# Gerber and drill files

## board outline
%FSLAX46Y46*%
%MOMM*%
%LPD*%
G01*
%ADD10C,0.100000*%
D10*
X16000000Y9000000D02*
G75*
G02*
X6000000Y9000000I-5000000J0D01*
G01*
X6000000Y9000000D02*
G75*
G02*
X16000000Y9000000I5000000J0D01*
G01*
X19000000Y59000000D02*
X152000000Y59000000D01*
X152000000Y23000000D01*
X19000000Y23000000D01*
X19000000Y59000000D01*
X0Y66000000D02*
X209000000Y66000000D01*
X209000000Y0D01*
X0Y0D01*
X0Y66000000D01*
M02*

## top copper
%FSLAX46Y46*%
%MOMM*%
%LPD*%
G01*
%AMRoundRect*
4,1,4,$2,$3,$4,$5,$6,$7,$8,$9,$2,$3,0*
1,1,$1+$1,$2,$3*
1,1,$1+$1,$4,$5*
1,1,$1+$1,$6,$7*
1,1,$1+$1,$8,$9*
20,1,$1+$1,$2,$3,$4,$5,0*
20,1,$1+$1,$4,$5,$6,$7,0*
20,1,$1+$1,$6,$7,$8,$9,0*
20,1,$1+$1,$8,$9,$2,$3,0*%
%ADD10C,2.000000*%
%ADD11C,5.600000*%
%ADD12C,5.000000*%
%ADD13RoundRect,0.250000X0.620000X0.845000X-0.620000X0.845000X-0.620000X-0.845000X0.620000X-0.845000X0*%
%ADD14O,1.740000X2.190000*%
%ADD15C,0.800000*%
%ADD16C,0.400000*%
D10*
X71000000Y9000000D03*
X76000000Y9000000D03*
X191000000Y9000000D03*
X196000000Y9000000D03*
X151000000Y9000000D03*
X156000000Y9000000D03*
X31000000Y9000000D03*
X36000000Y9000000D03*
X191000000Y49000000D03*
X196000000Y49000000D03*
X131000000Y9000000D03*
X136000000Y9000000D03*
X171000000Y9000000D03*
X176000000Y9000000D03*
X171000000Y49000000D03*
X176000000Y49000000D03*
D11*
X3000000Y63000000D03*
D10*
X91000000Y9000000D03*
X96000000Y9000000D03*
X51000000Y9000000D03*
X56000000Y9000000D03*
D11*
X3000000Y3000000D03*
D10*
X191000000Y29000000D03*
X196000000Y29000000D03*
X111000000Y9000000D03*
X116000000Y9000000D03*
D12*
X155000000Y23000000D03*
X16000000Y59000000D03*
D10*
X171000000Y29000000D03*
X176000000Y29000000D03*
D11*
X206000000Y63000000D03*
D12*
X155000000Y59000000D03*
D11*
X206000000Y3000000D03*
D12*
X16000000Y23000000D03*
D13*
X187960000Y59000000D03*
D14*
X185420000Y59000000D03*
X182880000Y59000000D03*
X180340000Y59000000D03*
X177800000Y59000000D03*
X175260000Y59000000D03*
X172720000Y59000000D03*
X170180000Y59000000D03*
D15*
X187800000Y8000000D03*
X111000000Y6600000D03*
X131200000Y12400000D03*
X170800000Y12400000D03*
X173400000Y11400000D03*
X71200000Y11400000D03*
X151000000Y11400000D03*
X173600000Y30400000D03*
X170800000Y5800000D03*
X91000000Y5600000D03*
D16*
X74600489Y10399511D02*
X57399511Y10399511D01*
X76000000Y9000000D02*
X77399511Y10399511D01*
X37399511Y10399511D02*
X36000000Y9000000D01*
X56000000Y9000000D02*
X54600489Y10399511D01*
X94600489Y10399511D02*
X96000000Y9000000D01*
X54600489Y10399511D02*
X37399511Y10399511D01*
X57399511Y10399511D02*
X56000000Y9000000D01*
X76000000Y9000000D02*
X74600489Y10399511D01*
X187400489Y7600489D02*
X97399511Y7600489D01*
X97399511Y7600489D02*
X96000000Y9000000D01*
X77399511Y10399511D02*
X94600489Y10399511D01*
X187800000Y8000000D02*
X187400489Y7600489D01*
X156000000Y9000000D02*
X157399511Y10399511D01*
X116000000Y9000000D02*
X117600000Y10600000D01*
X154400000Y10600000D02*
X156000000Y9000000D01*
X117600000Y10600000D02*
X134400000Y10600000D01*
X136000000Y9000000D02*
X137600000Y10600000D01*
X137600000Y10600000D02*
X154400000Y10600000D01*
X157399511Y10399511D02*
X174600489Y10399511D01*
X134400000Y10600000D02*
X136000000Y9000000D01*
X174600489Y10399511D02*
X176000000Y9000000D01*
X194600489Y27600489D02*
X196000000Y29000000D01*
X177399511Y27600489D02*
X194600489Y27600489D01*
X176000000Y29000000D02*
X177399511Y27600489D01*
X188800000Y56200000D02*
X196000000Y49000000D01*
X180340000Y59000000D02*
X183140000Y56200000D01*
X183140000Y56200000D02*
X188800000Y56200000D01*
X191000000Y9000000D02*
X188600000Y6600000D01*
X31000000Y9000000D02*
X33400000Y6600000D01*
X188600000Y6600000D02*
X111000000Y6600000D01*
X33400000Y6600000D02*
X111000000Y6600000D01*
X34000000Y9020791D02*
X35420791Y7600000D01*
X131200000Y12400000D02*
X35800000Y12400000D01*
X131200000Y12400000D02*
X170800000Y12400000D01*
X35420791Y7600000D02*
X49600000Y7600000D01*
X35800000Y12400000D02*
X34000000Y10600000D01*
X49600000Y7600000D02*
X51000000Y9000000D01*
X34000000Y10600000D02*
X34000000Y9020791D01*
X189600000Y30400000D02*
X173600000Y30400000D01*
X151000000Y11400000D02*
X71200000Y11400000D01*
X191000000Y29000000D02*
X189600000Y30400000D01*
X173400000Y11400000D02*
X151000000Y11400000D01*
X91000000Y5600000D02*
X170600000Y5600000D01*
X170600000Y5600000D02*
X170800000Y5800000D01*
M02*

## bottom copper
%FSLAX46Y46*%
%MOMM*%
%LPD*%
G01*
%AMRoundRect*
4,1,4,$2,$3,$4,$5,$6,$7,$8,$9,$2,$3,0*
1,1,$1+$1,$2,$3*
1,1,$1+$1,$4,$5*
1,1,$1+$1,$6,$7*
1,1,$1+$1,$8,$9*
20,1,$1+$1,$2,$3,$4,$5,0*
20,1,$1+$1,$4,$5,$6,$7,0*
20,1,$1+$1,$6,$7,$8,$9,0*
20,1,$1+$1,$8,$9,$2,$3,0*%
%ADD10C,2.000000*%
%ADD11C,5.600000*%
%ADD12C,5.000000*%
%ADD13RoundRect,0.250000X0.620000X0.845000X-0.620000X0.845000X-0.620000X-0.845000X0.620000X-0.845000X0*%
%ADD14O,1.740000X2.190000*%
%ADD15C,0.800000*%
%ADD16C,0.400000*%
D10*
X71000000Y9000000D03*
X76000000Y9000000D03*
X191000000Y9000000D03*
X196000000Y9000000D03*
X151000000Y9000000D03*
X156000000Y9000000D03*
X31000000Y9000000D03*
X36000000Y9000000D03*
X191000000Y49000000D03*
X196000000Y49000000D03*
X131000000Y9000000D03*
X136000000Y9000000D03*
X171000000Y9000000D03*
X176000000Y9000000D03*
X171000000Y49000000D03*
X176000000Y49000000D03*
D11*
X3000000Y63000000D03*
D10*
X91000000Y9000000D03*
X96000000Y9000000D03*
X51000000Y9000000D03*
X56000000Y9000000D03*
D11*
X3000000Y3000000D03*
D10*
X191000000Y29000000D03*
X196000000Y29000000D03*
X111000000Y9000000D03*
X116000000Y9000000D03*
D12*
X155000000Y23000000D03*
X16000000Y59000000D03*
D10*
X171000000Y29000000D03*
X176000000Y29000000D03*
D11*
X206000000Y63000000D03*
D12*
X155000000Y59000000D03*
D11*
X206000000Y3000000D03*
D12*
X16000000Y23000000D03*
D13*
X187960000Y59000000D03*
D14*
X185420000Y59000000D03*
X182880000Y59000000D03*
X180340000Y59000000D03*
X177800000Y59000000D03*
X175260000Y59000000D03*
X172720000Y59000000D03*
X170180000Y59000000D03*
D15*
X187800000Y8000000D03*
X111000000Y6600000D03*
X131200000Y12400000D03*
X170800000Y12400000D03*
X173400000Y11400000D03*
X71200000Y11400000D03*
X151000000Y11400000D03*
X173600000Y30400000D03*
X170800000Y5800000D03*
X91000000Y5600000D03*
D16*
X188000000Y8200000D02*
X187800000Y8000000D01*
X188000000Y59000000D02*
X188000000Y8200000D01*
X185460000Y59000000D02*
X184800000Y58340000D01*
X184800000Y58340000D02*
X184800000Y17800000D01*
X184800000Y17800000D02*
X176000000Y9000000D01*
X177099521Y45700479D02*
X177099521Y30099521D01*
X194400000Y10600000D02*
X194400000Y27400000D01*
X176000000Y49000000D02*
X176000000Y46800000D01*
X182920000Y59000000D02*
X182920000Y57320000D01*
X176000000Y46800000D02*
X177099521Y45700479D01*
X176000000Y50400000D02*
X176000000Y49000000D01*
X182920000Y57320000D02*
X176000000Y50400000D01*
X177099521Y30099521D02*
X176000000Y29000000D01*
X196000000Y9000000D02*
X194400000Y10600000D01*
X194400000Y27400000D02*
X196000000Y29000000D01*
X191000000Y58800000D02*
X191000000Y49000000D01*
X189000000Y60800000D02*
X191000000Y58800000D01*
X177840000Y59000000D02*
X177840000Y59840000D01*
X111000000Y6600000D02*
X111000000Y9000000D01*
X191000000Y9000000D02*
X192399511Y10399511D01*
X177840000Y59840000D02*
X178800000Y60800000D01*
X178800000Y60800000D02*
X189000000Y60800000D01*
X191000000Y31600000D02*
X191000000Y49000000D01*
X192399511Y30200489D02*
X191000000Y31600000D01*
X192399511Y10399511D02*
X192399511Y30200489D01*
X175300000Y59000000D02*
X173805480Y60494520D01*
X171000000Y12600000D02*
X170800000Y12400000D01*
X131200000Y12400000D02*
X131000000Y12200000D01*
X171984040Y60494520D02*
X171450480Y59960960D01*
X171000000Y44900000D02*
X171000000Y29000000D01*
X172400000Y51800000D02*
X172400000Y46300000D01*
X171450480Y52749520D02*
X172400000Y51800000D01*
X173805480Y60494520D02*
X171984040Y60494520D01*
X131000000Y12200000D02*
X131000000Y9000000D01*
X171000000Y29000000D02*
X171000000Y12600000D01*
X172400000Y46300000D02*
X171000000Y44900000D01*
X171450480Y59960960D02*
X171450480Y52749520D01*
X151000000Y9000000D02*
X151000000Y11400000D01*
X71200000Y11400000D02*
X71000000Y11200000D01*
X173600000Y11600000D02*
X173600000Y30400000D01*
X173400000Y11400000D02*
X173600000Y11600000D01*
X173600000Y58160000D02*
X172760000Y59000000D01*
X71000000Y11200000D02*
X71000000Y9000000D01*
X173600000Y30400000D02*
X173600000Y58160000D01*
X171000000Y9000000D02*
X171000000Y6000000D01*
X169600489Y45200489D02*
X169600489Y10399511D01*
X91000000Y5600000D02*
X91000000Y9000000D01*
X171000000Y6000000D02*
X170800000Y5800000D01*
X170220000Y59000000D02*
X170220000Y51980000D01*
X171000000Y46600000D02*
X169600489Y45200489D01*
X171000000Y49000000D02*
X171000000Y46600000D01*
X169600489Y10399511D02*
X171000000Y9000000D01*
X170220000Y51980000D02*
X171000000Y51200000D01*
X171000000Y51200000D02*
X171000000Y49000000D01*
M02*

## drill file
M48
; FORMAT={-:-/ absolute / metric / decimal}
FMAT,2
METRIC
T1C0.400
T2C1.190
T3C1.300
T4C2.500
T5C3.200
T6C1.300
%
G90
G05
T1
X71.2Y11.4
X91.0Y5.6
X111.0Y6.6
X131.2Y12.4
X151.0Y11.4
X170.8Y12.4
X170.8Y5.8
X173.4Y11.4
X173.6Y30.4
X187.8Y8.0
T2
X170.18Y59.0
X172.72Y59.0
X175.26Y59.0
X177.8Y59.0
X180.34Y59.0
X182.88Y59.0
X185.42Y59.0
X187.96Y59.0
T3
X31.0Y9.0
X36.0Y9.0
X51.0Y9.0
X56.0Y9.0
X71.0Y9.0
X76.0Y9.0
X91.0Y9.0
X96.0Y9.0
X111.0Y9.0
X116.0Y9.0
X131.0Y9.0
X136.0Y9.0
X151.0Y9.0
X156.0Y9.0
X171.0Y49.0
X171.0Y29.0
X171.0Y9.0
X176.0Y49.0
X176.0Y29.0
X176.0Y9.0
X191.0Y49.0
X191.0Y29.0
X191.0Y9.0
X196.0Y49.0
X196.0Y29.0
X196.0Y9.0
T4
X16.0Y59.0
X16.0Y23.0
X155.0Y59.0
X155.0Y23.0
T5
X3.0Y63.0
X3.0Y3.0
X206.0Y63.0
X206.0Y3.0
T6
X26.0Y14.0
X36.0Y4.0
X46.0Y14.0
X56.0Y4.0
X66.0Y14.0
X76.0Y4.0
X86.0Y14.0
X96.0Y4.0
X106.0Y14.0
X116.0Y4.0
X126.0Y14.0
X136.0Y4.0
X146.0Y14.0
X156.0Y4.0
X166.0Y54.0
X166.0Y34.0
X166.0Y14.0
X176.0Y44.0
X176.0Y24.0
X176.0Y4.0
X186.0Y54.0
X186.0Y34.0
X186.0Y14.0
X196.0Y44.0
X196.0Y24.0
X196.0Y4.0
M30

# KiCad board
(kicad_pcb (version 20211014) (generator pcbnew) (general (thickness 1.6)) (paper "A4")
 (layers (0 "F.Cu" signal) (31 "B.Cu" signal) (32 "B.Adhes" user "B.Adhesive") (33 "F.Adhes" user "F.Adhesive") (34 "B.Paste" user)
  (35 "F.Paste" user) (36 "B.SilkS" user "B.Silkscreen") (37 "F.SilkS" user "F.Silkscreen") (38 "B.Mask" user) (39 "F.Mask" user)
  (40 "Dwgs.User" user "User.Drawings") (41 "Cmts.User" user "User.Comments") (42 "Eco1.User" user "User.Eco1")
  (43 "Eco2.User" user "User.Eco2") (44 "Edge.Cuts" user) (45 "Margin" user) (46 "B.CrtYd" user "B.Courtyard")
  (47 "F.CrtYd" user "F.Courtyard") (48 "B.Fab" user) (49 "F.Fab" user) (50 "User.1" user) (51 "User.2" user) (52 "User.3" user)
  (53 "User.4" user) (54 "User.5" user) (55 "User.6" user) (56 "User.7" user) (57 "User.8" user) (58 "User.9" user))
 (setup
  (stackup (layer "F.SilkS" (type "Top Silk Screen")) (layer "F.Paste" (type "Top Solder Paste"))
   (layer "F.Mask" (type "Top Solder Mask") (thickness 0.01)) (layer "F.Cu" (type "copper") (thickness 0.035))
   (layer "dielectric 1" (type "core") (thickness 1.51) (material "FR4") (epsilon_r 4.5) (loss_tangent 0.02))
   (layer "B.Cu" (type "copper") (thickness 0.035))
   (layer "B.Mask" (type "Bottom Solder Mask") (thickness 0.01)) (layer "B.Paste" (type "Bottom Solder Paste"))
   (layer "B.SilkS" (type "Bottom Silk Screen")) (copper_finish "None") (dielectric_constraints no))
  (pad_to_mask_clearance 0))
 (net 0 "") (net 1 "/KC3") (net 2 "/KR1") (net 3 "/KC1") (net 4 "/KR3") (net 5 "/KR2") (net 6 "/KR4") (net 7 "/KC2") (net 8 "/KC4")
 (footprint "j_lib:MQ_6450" (layer "F.Cu") (at 71 -9)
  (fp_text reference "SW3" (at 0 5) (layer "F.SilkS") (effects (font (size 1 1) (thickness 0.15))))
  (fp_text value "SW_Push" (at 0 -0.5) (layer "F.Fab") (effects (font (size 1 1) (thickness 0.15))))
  (pad "" np_thru_hole circle locked (at -5 -5) (size 1.3 1.3) (drill 1.3) (layers *.Cu *.Mask))
  (pad "" np_thru_hole circle locked (at 5 5) (size 1.3 1.3) (drill 1.3) (layers *.Cu *.Mask))
  (pad "1" thru_hole circle locked (at 0 0) (size 2 2) (drill 1.3) (layers *.Cu *.Mask) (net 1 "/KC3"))
  (pad "2" thru_hole circle locked (at 5 0) (size 2 2) (drill 1.3) (layers *.Cu *.Mask) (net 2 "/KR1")))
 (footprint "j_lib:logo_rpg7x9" (layer "F.Cu") (at 158.2 -39.4)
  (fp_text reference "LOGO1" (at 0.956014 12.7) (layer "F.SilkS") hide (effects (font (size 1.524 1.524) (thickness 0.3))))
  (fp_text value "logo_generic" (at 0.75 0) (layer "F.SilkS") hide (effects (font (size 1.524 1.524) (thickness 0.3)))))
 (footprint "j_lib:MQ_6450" (layer "F.Cu") (at 191 -9)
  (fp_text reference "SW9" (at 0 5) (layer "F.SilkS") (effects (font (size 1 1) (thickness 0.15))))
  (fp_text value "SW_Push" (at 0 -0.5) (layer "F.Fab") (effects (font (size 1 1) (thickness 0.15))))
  (pad "" np_thru_hole circle locked (at 5 5) (size 1.3 1.3) (drill 1.3) (layers *.Cu *.Mask))
  (pad "" np_thru_hole circle locked (at -5 -5) (size 1.3 1.3) (drill 1.3) (layers *.Cu *.Mask))
  (pad "1" thru_hole circle locked (at 0 0) (size 2 2) (drill 1.3) (layers *.Cu *.Mask) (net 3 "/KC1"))
  (pad "2" thru_hole circle locked (at 5 0) (size 2 2) (drill 1.3) (layers *.Cu *.Mask) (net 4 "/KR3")))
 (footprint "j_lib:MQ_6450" (layer "F.Cu") (at 151 -9)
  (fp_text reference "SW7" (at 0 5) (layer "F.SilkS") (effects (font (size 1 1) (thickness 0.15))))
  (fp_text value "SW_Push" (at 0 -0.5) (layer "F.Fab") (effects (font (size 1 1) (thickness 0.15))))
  (pad "" np_thru_hole circle locked (at 5 5) (size 1.3 1.3) (drill 1.3) (layers *.Cu *.Mask))
  (pad "" np_thru_hole circle locked (at -5 -5) (size 1.3 1.3) (drill 1.3) (layers *.Cu *.Mask))
  (pad "1" thru_hole circle locked (at 0 0) (size 2 2) (drill 1.3) (layers *.Cu *.Mask) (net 1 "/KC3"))
  (pad "2" thru_hole circle locked (at 5 0) (size 2 2) (drill 1.3) (layers *.Cu *.Mask) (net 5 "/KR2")))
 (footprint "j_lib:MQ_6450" (layer "F.Cu") (at 31 -9)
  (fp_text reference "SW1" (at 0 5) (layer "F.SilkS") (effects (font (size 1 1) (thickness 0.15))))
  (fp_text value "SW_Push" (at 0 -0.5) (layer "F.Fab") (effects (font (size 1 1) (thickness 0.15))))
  (pad "" np_thru_hole circle locked (at 5 5) (size 1.3 1.3) (drill 1.3) (layers *.Cu *.Mask))
  (pad "" np_thru_hole circle locked (at -5 -5) (size 1.3 1.3) (drill 1.3) (layers *.Cu *.Mask))
  (pad "1" thru_hole circle locked (at 0 0) (size 2 2) (drill 1.3) (layers *.Cu *.Mask) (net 3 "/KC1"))
  (pad "2" thru_hole circle locked (at 5 0) (size 2 2) (drill 1.3) (layers *.Cu *.Mask) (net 2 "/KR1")))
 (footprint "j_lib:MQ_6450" (layer "F.Cu") (at 191 -49)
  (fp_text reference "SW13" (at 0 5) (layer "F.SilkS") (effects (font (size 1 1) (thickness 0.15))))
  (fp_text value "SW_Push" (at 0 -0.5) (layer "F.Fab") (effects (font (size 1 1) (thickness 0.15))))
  (pad "" np_thru_hole circle locked (at -5 -5) (size 1.3 1.3) (drill 1.3) (layers *.Cu *.Mask))
  (pad "" np_thru_hole circle locked (at 5 5) (size 1.3 1.3) (drill 1.3) (layers *.Cu *.Mask))
  (pad "1" thru_hole circle locked (at 0 0) (size 2 2) (drill 1.3) (layers *.Cu *.Mask) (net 3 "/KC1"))
  (pad "2" thru_hole circle locked (at 5 0) (size 2 2) (drill 1.3) (layers *.Cu *.Mask) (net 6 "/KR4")))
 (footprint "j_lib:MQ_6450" (layer "F.Cu") (at 131 -9)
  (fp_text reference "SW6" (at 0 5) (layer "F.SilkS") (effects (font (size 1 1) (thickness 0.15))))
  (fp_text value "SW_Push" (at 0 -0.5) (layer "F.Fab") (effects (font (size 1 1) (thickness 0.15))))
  (pad "" np_thru_hole circle locked (at 5 5) (size 1.3 1.3) (drill 1.3) (layers *.Cu *.Mask))
  (pad "" np_thru_hole circle locked (at -5 -5) (size 1.3 1.3) (drill 1.3) (layers *.Cu *.Mask))
  (pad "1" thru_hole circle locked (at 0 0) (size 2 2) (drill 1.3) (layers *.Cu *.Mask) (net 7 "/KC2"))
  (pad "2" thru_hole circle locked (at 5 0) (size 2 2) (drill 1.3) (layers *.Cu *.Mask) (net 5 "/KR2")))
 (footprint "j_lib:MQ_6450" (layer "F.Cu") (at 171 -9)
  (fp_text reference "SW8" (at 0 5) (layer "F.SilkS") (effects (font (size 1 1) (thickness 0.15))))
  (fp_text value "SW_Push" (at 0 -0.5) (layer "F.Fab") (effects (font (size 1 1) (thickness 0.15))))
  (pad "" np_thru_hole circle locked (at -5 -5) (size 1.3 1.3) (drill 1.3) (layers *.Cu *.Mask))
  (pad "" np_thru_hole circle locked (at 5 5) (size 1.3 1.3) (drill 1.3) (layers *.Cu *.Mask))
  (pad "1" thru_hole circle locked (at 0 0) (size 2 2) (drill 1.3) (layers *.Cu *.Mask) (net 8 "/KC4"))
  (pad "2" thru_hole circle locked (at 5 0) (size 2 2) (drill 1.3) (layers *.Cu *.Mask) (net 5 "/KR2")))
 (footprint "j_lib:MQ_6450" (layer "F.Cu") (at 171 -49)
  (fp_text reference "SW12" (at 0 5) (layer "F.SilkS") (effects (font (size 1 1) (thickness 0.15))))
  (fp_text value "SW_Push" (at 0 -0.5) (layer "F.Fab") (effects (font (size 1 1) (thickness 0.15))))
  (pad "" np_thru_hole circle locked (at 5 5) (size 1.3 1.3) (drill 1.3) (layers *.Cu *.Mask))
  (pad "" np_thru_hole circle locked (at -5 -5) (size 1.3 1.3) (drill 1.3) (layers *.Cu *.Mask))
  (pad "1" thru_hole circle locked (at 0 0) (size 2 2) (drill 1.3) (layers *.Cu *.Mask) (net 8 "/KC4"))
  (pad "2" thru_hole circle locked (at 5 0) (size 2 2) (drill 1.3) (layers *.Cu *.Mask) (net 4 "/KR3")))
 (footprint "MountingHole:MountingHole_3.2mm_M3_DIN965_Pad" (layer "F.Cu") (at 3 -63)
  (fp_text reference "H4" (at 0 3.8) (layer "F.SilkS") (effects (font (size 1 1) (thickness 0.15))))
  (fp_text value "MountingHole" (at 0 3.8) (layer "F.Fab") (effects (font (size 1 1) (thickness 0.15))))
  (pad "1" thru_hole circle locked (at 0 0) (size 5.6 5.6) (drill 3.2) (layers *.Cu *.Mask)))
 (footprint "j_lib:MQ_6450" (layer "F.Cu") (at 91 -9)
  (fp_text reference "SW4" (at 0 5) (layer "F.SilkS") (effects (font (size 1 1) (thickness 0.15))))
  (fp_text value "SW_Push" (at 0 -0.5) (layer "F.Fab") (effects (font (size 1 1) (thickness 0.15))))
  (pad "" np_thru_hole circle locked (at -5 -5) (size 1.3 1.3) (drill 1.3) (layers *.Cu *.Mask))
  (pad "" np_thru_hole circle locked (at 5 5) (size 1.3 1.3) (drill 1.3) (layers *.Cu *.Mask))
  (pad "1" thru_hole circle locked (at 0 0) (size 2 2) (drill 1.3) (layers *.Cu *.Mask) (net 8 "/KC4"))
  (pad "2" thru_hole circle locked (at 5 0) (size 2 2) (drill 1.3) (layers *.Cu *.Mask) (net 2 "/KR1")))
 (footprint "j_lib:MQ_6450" (layer "F.Cu") (at 51 -9)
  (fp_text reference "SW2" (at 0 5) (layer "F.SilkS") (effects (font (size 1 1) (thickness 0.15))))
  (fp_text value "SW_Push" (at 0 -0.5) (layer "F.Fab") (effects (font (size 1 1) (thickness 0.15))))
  (pad "" np_thru_hole circle locked (at -5 -5) (size 1.3 1.3) (drill 1.3) (layers *.Cu *.Mask))
  (pad "" np_thru_hole circle locked (at 5 5) (size 1.3 1.3) (drill 1.3) (layers *.Cu *.Mask))
  (pad "1" thru_hole circle locked (at 0 0) (size 2 2) (drill 1.3) (layers *.Cu *.Mask) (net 7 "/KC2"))
  (pad "2" thru_hole circle locked (at 5 0) (size 2 2) (drill 1.3) (layers *.Cu *.Mask) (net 2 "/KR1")))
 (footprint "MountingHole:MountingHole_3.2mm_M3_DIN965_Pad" (layer "F.Cu") (at 3 -3)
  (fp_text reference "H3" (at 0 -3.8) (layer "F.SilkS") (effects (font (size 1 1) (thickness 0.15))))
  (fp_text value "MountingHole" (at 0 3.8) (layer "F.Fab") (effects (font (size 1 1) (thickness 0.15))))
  (pad "1" thru_hole circle locked (at 0 0) (size 5.6 5.6) (drill 3.2) (layers *.Cu *.Mask)))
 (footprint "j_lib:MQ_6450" (layer "F.Cu") (at 191 -29)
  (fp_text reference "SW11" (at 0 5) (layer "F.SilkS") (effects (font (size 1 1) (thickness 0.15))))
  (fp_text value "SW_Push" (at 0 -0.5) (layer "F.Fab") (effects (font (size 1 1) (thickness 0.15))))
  (pad "" np_thru_hole circle locked (at 5 5) (size 1.3 1.3) (drill 1.3) (layers *.Cu *.Mask))
  (pad "" np_thru_hole circle locked (at -5 -5) (size 1.3 1.3) (drill 1.3) (layers *.Cu *.Mask))
  (pad "1" thru_hole circle locked (at 0 0) (size 2 2) (drill 1.3) (layers *.Cu *.Mask) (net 1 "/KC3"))
  (pad "2" thru_hole circle locked (at 5 0) (size 2 2) (drill 1.3) (layers *.Cu *.Mask) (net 4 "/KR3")))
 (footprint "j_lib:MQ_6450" (layer "F.Cu") (at 111 -9)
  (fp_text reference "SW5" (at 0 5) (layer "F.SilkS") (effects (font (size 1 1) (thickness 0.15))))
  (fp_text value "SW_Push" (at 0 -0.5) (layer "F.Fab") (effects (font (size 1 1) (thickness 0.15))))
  (pad "" np_thru_hole circle locked (at 5 5) (size 1.3 1.3) (drill 1.3) (layers *.Cu *.Mask))
  (pad "" np_thru_hole circle locked (at -5 -5) (size 1.3 1.3) (drill 1.3) (layers *.Cu *.Mask))
  (pad "1" thru_hole circle locked (at 0 0) (size 2 2) (drill 1.3) (layers *.Cu *.Mask) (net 3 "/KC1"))
  (pad "2" thru_hole circle locked (at 5 0) (size 2 2) (drill 1.3) (layers *.Cu *.Mask) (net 5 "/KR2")))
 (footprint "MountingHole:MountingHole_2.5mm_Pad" (layer "F.Cu") (at 155 -23)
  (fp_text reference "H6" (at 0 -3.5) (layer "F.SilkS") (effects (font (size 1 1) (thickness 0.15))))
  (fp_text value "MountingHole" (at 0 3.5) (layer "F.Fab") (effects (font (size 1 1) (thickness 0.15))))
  (pad "1" thru_hole circle locked (at 0 0) (size 5 5) (drill 2.5) (layers *.Cu *.Mask)))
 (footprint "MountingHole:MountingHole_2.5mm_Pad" (layer "F.Cu") (at 16 -59)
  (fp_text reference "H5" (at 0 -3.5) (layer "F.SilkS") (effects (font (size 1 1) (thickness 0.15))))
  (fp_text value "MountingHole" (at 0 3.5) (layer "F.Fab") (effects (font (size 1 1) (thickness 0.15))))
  (pad "1" thru_hole circle locked (at 0 0) (size 5 5) (drill 2.5) (layers *.Cu *.Mask)))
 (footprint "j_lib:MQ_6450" (layer "F.Cu") (at 171 -29)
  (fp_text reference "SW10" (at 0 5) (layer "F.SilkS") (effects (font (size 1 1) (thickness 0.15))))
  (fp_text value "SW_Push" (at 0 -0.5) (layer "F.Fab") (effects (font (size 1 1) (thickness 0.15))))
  (pad "" np_thru_hole circle locked (at 5 5) (size 1.3 1.3) (drill 1.3) (layers *.Cu *.Mask))
  (pad "" np_thru_hole circle locked (at -5 -5) (size 1.3 1.3) (drill 1.3) (layers *.Cu *.Mask))
  (pad "1" thru_hole circle locked (at 0 0) (size 2 2) (drill 1.3) (layers *.Cu *.Mask) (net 7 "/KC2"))
  (pad "2" thru_hole circle locked (at 5 0) (size 2 2) (drill 1.3) (layers *.Cu *.Mask) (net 4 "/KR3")))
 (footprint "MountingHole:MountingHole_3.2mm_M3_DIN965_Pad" (layer "F.Cu") (at 206 -63)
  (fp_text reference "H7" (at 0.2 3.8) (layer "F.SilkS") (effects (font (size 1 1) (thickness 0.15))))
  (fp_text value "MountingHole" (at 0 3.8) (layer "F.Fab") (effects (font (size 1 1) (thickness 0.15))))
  (pad "1" thru_hole circle locked (at 0 0) (size 5.6 5.6) (drill 3.2) (layers *.Cu *.Mask)))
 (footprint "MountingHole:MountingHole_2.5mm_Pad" (layer "F.Cu") (at 155 -59)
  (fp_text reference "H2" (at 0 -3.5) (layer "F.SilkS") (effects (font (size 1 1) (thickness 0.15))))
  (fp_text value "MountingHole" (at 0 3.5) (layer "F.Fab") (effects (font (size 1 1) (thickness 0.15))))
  (pad "1" thru_hole circle locked (at 0 0) (size 5 5) (drill 2.5) (layers *.Cu *.Mask)))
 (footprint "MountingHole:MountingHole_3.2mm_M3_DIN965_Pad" (layer "F.Cu") (at 206 -3)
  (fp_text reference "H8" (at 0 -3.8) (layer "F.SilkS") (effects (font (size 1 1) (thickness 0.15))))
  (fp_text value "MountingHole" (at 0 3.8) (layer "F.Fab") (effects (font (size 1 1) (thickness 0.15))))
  (pad "1" thru_hole circle locked (at 0 0) (size 5.6 5.6) (drill 3.2) (layers *.Cu *.Mask)))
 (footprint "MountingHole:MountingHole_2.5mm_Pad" (layer "F.Cu") (at 16 -23)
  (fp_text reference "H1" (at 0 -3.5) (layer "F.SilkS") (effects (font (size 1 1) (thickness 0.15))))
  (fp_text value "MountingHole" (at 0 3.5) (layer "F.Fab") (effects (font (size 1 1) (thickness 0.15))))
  (pad "1" thru_hole circle locked (at 0 0) (size 5 5) (drill 2.5) (layers *.Cu *.Mask)))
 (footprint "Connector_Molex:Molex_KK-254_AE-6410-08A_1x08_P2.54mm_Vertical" (layer "B.Cu") (at 187.96 -59 180)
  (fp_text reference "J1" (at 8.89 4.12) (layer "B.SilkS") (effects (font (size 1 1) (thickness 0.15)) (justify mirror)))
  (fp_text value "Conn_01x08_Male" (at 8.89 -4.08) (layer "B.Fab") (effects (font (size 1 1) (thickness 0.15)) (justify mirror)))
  (pad "1" thru_hole roundrect locked (at 0 0 180) (size 1.74 2.19) (drill 1.19) (layers *.Cu *.Mask) (roundrect_rratio 0.1436781609)
   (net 2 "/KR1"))
  (pad "2" thru_hole oval locked (at 2.54 0 180) (size 1.74 2.19) (drill 1.19) (layers *.Cu *.Mask) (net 5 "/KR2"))
  (pad "3" thru_hole oval locked (at 5.08 0 180) (size 1.74 2.19) (drill 1.19) (layers *.Cu *.Mask) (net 4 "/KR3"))
  (pad "4" thru_hole oval locked (at 7.62 0 180) (size 1.74 2.19) (drill 1.19) (layers *.Cu *.Mask) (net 6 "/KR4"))
  (pad "5" thru_hole oval locked (at 10.16 0 180) (size 1.74 2.19) (drill 1.19) (layers *.Cu *.Mask) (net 3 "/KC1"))
  (pad "6" thru_hole oval locked (at 12.7 0 180) (size 1.74 2.19) (drill 1.19) (layers *.Cu *.Mask) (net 7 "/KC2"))
  (pad "7" thru_hole oval locked (at 15.24 0 180) (size 1.74 2.19) (drill 1.19) (layers *.Cu *.Mask) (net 1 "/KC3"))
  (pad "8" thru_hole oval locked (at 17.78 0 180) (size 1.74 2.19) (drill 1.19) (layers *.Cu *.Mask) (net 8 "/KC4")))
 (gr_circle (center 11 -9) (end 16 -9) (layer "Edge.Cuts") (width 0.1) (fill none))
 (gr_rect (start 19 -23) (end 152 -59) (layer "Edge.Cuts") (width 0.1) (fill none))
 (gr_rect (start 0 0) (end 209 -66) (layer "Edge.Cuts") (width 0.1) (fill none))
 (segment (start 74.600489 -10.399511) (end 57.399511 -10.399511) (width 0.4) (layer "F.Cu") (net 2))
 (segment (start 76 -9) (end 77.399511 -10.399511) (width 0.4) (layer "F.Cu") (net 2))
 (segment (start 37.399511 -10.399511) (end 36 -9) (width 0.4) (layer "F.Cu") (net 2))
 (segment (start 56 -9) (end 54.600489 -10.399511) (width 0.4) (layer "F.Cu") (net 2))
 (segment (start 94.600489 -10.399511) (end 96 -9) (width 0.4) (layer "F.Cu") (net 2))
 (segment (start 54.600489 -10.399511) (end 37.399511 -10.399511) (width 0.4) (layer "F.Cu") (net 2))
 (segment (start 57.399511 -10.399511) (end 56 -9) (width 0.4) (layer "F.Cu") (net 2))
 (segment (start 76 -9) (end 74.600489 -10.399511) (width 0.4) (layer "F.Cu") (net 2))
 (segment (start 187.400489 -7.600489) (end 97.399511 -7.600489) (width 0.4) (layer "F.Cu") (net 2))
 (segment (start 97.399511 -7.600489) (end 96 -9) (width 0.4) (layer "F.Cu") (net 2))
 (segment (start 77.399511 -10.399511) (end 94.600489 -10.399511) (width 0.4) (layer "F.Cu") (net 2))
 (segment (start 187.8 -8) (end 187.400489 -7.600489) (width 0.4) (layer "F.Cu") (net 2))
 (via (at 187.8 -8) (size 0.8) (drill 0.4) (layers "F.Cu" "B.Cu") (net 2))
 (segment (start 188 -8.2) (end 187.8 -8) (width 0.4) (layer "B.Cu") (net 2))
 (segment (start 188 -59) (end 188 -8.2) (width 0.4) (layer "B.Cu") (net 2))
 (segment (start 156 -9) (end 157.399511 -10.399511) (width 0.4) (layer "F.Cu") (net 5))
 (segment (start 116 -9) (end 117.6 -10.6) (width 0.4) (layer "F.Cu") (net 5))
 (segment (start 154.4 -10.6) (end 156 -9) (width 0.4) (layer "F.Cu") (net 5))
 (segment (start 117.6 -10.6) (end 134.4 -10.6) (width 0.4) (layer "F.Cu") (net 5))
 (segment (start 136 -9) (end 137.6 -10.6) (width 0.4) (layer "F.Cu") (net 5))
 (segment (start 137.6 -10.6) (end 154.4 -10.6) (width 0.4) (layer "F.Cu") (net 5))
 (segment (start 157.399511 -10.399511) (end 174.600489 -10.399511) (width 0.4) (layer "F.Cu") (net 5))
 (segment (start 134.4 -10.6) (end 136 -9) (width 0.4) (layer "F.Cu") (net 5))
 (segment (start 174.600489 -10.399511) (end 176 -9) (width 0.4) (layer "F.Cu") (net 5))
 (segment (start 185.46 -59) (end 184.8 -58.34) (width 0.4) (layer "B.Cu") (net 5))
 (segment (start 184.8 -58.34) (end 184.8 -17.8) (width 0.4) (layer "B.Cu") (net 5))
 (segment (start 184.8 -17.8) (end 176 -9) (width 0.4) (layer "B.Cu") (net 5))
 (segment (start 194.600489 -27.600489) (end 196 -29) (width 0.4) (layer "F.Cu") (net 4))
 (segment (start 177.399511 -27.600489) (end 194.600489 -27.600489) (width 0.4) (layer "F.Cu") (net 4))
 (segment (start 176 -29) (end 177.399511 -27.600489) (width 0.4) (layer "F.Cu") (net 4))
 (segment (start 177.099521 -45.700479) (end 177.099521 -30.099521) (width 0.4) (layer "B.Cu") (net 4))
 (segment (start 194.4 -10.6) (end 194.4 -27.4) (width 0.4) (layer "B.Cu") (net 4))
 (segment (start 176 -49) (end 176 -46.8) (width 0.4) (layer "B.Cu") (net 4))
 (segment (start 182.92 -59) (end 182.92 -57.32) (width 0.4) (layer "B.Cu") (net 4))
 (segment (start 176 -46.8) (end 177.099521 -45.700479) (width 0.4) (layer "B.Cu") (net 4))
 (segment (start 176 -50.4) (end 176 -49) (width 0.4) (layer "B.Cu") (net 4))
 (segment (start 182.92 -57.32) (end 176 -50.4) (width 0.4) (layer "B.Cu") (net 4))
 (segment (start 177.099521 -30.099521) (end 176 -29) (width 0.4) (layer "B.Cu") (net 4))
 (segment (start 196 -9) (end 194.4 -10.6) (width 0.4) (layer "B.Cu") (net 4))
 (segment (start 194.4 -27.4) (end 196 -29) (width 0.4) (layer "B.Cu") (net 4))
 (segment (start 188.8 -56.2) (end 196 -49) (width 0.4) (layer "F.Cu") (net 6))
 (segment (start 180.34 -59) (end 183.14 -56.2) (width 0.4) (layer "F.Cu") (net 6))
 (segment (start 183.14 -56.2) (end 188.8 -56.2) (width 0.4) (layer "F.Cu") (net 6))
 (segment (start 191 -9) (end 188.6 -6.6) (width 0.4) (layer "F.Cu") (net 3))
 (segment (start 31 -9) (end 33.4 -6.6) (width 0.4) (layer "F.Cu") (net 3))
 (segment (start 188.6 -6.6) (end 111 -6.6) (width 0.4) (layer "F.Cu") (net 3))
 (segment (start 33.4 -6.6) (end 111 -6.6) (width 0.4) (layer "F.Cu") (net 3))
 (via (at 111 -6.6) (size 0.8) (drill 0.4) (layers "F.Cu" "B.Cu") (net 3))
 (segment (start 191 -58.8) (end 191 -49) (width 0.4) (layer "B.Cu") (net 3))
 (segment (start 189 -60.8) (end 191 -58.8) (width 0.4) (layer "B.Cu") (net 3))
 (segment (start 177.84 -59) (end 177.84 -59.84) (width 0.4) (layer "B.Cu") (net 3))
 (segment (start 111 -6.6) (end 111 -9) (width 0.4) (layer "B.Cu") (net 3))
 (segment (start 191 -9) (end 192.399511 -10.399511) (width 0.4) (layer "B.Cu") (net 3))
 (segment (start 177.84 -59.84) (end 178.8 -60.8) (width 0.4) (layer "B.Cu") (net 3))
 (segment (start 178.8 -60.8) (end 189 -60.8) (width 0.4) (layer "B.Cu") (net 3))
 (segment (start 191 -31.6) (end 191 -49) (width 0.4) (layer "B.Cu") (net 3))
 (segment (start 192.399511 -30.200489) (end 191 -31.6) (width 0.4) (layer "B.Cu") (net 3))
 (segment (start 192.399511 -10.399511) (end 192.399511 -30.200489) (width 0.4) (layer "B.Cu") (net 3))
 (segment (start 34 -9.020791) (end 35.420791 -7.6) (width 0.4) (layer "F.Cu") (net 7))
 (segment (start 131.2 -12.4) (end 35.8 -12.4) (width 0.4) (layer "F.Cu") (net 7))
 (segment (start 131.2 -12.4) (end 170.8 -12.4) (width 0.4) (layer "F.Cu") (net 7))
 (segment (start 35.420791 -7.6) (end 49.6 -7.6) (width 0.4) (layer "F.Cu") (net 7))
 (segment (start 35.8 -12.4) (end 34 -10.6) (width 0.4) (layer "F.Cu") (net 7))
 (segment (start 49.6 -7.6) (end 51 -9) (width 0.4) (layer "F.Cu") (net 7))
 (segment (start 34 -10.6) (end 34 -9.020791) (width 0.4) (layer "F.Cu") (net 7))
 (via (at 131.2 -12.4) (size 0.8) (drill 0.4) (layers "F.Cu" "B.Cu") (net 7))
 (via (at 170.8 -12.4) (size 0.8) (drill 0.4) (layers "F.Cu" "B.Cu") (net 7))
 (segment (start 175.3 -59) (end 173.80548 -60.49452) (width 0.4) (layer "B.Cu") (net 7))
 (segment (start 171 -12.6) (end 170.8 -12.4) (width 0.4) (layer "B.Cu") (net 7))
 (segment (start 131.2 -12.4) (end 131 -12.2) (width 0.4) (layer "B.Cu") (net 7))
 (segment (start 171.98404 -60.49452) (end 171.45048 -59.96096) (width 0.4) (layer "B.Cu") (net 7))
 (segment (start 171 -44.9) (end 171 -29) (width 0.4) (layer "B.Cu") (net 7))
 (segment (start 172.4 -51.8) (end 172.4 -46.3) (width 0.4) (layer "B.Cu") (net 7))
 (segment (start 171.45048 -52.74952) (end 172.4 -51.8) (width 0.4) (layer "B.Cu") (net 7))
 (segment (start 173.80548 -60.49452) (end 171.98404 -60.49452) (width 0.4) (layer "B.Cu") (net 7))
 (segment (start 131 -12.2) (end 131 -9) (width 0.4) (layer "B.Cu") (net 7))
 (segment (start 171 -29) (end 171 -12.6) (width 0.4) (layer "B.Cu") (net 7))
 (segment (start 172.4 -46.3) (end 171 -44.9) (width 0.4) (layer "B.Cu") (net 7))
 (segment (start 171.45048 -59.96096) (end 171.45048 -52.74952) (width 0.4) (layer "B.Cu") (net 7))
 (segment (start 189.6 -30.4) (end 173.6 -30.4) (width 0.4) (layer "F.Cu") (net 1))
 (segment (start 151 -11.4) (end 71.2 -11.4) (width 0.4) (layer "F.Cu") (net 1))
 (segment (start 191 -29) (end 189.6 -30.4) (width 0.4) (layer "F.Cu") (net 1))
 (segment (start 173.4 -11.4) (end 151 -11.4) (width 0.4) (layer "F.Cu") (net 1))
 (via (at 173.4 -11.4) (size 0.8) (drill 0.4) (layers "F.Cu" "B.Cu") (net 1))
 (via (at 71.2 -11.4) (size 0.8) (drill 0.4) (layers "F.Cu" "B.Cu") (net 1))
 (via (at 151 -11.4) (size 0.8) (drill 0.4) (layers "F.Cu" "B.Cu") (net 1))
 (via (at 173.6 -30.4) (size 0.8) (drill 0.4) (layers "F.Cu" "B.Cu") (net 1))
 (segment (start 151 -9) (end 151 -11.4) (width 0.4) (layer "B.Cu") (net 1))
 (segment (start 71.2 -11.4) (end 71 -11.2) (width 0.4) (layer "B.Cu") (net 1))
 (segment (start 173.6 -11.6) (end 173.6 -30.4) (width 0.4) (layer "B.Cu") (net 1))
 (segment (start 173.4 -11.4) (end 173.6 -11.6) (width 0.4) (layer "B.Cu") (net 1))
 (segment (start 173.6 -58.16) (end 172.76 -59) (width 0.4) (layer "B.Cu") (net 1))
 (segment (start 71 -11.2) (end 71 -9) (width 0.4) (layer "B.Cu") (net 1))
 (segment (start 173.6 -30.4) (end 173.6 -58.16) (width 0.4) (layer "B.Cu") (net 1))
 (segment (start 91 -5.6) (end 170.6 -5.6) (width 0.4) (layer "F.Cu") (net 8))
 (segment (start 170.6 -5.6) (end 170.8 -5.8) (width 0.4) (layer "F.Cu") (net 8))
 (via (at 170.8 -5.8) (size 0.8) (drill 0.4) (layers "F.Cu" "B.Cu") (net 8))
 (via (at 91 -5.6) (size 0.8) (drill 0.4) (layers "F.Cu" "B.Cu") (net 8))
 (segment (start 171 -9) (end 171 -6) (width 0.4) (layer "B.Cu") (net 8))
 (segment (start 169.600489 -45.200489) (end 169.600489 -10.399511) (width 0.4) (layer "B.Cu") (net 8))
 (segment (start 91 -5.6) (end 91 -9) (width 0.4) (layer "B.Cu") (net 8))
 (segment (start 171 -6) (end 170.8 -5.8) (width 0.4) (layer "B.Cu") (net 8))
 (segment (start 170.22 -59) (end 170.22 -51.98) (width 0.4) (layer "B.Cu") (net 8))
 (segment (start 171 -46.6) (end 169.600489 -45.200489) (width 0.4) (layer "B.Cu") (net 8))
 (segment (start 171 -49) (end 171 -46.6) (width 0.4) (layer "B.Cu") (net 8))
 (segment (start 169.600489 -10.399511) (end 171 -9) (width 0.4) (layer "B.Cu") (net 8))
 (segment (start 170.22 -51.98) (end 171 -51.2) (width 0.4) (layer "B.Cu") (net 8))
 (segment (start 171 -51.2) (end 171 -49) (width 0.4) (layer "B.Cu") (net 8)))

